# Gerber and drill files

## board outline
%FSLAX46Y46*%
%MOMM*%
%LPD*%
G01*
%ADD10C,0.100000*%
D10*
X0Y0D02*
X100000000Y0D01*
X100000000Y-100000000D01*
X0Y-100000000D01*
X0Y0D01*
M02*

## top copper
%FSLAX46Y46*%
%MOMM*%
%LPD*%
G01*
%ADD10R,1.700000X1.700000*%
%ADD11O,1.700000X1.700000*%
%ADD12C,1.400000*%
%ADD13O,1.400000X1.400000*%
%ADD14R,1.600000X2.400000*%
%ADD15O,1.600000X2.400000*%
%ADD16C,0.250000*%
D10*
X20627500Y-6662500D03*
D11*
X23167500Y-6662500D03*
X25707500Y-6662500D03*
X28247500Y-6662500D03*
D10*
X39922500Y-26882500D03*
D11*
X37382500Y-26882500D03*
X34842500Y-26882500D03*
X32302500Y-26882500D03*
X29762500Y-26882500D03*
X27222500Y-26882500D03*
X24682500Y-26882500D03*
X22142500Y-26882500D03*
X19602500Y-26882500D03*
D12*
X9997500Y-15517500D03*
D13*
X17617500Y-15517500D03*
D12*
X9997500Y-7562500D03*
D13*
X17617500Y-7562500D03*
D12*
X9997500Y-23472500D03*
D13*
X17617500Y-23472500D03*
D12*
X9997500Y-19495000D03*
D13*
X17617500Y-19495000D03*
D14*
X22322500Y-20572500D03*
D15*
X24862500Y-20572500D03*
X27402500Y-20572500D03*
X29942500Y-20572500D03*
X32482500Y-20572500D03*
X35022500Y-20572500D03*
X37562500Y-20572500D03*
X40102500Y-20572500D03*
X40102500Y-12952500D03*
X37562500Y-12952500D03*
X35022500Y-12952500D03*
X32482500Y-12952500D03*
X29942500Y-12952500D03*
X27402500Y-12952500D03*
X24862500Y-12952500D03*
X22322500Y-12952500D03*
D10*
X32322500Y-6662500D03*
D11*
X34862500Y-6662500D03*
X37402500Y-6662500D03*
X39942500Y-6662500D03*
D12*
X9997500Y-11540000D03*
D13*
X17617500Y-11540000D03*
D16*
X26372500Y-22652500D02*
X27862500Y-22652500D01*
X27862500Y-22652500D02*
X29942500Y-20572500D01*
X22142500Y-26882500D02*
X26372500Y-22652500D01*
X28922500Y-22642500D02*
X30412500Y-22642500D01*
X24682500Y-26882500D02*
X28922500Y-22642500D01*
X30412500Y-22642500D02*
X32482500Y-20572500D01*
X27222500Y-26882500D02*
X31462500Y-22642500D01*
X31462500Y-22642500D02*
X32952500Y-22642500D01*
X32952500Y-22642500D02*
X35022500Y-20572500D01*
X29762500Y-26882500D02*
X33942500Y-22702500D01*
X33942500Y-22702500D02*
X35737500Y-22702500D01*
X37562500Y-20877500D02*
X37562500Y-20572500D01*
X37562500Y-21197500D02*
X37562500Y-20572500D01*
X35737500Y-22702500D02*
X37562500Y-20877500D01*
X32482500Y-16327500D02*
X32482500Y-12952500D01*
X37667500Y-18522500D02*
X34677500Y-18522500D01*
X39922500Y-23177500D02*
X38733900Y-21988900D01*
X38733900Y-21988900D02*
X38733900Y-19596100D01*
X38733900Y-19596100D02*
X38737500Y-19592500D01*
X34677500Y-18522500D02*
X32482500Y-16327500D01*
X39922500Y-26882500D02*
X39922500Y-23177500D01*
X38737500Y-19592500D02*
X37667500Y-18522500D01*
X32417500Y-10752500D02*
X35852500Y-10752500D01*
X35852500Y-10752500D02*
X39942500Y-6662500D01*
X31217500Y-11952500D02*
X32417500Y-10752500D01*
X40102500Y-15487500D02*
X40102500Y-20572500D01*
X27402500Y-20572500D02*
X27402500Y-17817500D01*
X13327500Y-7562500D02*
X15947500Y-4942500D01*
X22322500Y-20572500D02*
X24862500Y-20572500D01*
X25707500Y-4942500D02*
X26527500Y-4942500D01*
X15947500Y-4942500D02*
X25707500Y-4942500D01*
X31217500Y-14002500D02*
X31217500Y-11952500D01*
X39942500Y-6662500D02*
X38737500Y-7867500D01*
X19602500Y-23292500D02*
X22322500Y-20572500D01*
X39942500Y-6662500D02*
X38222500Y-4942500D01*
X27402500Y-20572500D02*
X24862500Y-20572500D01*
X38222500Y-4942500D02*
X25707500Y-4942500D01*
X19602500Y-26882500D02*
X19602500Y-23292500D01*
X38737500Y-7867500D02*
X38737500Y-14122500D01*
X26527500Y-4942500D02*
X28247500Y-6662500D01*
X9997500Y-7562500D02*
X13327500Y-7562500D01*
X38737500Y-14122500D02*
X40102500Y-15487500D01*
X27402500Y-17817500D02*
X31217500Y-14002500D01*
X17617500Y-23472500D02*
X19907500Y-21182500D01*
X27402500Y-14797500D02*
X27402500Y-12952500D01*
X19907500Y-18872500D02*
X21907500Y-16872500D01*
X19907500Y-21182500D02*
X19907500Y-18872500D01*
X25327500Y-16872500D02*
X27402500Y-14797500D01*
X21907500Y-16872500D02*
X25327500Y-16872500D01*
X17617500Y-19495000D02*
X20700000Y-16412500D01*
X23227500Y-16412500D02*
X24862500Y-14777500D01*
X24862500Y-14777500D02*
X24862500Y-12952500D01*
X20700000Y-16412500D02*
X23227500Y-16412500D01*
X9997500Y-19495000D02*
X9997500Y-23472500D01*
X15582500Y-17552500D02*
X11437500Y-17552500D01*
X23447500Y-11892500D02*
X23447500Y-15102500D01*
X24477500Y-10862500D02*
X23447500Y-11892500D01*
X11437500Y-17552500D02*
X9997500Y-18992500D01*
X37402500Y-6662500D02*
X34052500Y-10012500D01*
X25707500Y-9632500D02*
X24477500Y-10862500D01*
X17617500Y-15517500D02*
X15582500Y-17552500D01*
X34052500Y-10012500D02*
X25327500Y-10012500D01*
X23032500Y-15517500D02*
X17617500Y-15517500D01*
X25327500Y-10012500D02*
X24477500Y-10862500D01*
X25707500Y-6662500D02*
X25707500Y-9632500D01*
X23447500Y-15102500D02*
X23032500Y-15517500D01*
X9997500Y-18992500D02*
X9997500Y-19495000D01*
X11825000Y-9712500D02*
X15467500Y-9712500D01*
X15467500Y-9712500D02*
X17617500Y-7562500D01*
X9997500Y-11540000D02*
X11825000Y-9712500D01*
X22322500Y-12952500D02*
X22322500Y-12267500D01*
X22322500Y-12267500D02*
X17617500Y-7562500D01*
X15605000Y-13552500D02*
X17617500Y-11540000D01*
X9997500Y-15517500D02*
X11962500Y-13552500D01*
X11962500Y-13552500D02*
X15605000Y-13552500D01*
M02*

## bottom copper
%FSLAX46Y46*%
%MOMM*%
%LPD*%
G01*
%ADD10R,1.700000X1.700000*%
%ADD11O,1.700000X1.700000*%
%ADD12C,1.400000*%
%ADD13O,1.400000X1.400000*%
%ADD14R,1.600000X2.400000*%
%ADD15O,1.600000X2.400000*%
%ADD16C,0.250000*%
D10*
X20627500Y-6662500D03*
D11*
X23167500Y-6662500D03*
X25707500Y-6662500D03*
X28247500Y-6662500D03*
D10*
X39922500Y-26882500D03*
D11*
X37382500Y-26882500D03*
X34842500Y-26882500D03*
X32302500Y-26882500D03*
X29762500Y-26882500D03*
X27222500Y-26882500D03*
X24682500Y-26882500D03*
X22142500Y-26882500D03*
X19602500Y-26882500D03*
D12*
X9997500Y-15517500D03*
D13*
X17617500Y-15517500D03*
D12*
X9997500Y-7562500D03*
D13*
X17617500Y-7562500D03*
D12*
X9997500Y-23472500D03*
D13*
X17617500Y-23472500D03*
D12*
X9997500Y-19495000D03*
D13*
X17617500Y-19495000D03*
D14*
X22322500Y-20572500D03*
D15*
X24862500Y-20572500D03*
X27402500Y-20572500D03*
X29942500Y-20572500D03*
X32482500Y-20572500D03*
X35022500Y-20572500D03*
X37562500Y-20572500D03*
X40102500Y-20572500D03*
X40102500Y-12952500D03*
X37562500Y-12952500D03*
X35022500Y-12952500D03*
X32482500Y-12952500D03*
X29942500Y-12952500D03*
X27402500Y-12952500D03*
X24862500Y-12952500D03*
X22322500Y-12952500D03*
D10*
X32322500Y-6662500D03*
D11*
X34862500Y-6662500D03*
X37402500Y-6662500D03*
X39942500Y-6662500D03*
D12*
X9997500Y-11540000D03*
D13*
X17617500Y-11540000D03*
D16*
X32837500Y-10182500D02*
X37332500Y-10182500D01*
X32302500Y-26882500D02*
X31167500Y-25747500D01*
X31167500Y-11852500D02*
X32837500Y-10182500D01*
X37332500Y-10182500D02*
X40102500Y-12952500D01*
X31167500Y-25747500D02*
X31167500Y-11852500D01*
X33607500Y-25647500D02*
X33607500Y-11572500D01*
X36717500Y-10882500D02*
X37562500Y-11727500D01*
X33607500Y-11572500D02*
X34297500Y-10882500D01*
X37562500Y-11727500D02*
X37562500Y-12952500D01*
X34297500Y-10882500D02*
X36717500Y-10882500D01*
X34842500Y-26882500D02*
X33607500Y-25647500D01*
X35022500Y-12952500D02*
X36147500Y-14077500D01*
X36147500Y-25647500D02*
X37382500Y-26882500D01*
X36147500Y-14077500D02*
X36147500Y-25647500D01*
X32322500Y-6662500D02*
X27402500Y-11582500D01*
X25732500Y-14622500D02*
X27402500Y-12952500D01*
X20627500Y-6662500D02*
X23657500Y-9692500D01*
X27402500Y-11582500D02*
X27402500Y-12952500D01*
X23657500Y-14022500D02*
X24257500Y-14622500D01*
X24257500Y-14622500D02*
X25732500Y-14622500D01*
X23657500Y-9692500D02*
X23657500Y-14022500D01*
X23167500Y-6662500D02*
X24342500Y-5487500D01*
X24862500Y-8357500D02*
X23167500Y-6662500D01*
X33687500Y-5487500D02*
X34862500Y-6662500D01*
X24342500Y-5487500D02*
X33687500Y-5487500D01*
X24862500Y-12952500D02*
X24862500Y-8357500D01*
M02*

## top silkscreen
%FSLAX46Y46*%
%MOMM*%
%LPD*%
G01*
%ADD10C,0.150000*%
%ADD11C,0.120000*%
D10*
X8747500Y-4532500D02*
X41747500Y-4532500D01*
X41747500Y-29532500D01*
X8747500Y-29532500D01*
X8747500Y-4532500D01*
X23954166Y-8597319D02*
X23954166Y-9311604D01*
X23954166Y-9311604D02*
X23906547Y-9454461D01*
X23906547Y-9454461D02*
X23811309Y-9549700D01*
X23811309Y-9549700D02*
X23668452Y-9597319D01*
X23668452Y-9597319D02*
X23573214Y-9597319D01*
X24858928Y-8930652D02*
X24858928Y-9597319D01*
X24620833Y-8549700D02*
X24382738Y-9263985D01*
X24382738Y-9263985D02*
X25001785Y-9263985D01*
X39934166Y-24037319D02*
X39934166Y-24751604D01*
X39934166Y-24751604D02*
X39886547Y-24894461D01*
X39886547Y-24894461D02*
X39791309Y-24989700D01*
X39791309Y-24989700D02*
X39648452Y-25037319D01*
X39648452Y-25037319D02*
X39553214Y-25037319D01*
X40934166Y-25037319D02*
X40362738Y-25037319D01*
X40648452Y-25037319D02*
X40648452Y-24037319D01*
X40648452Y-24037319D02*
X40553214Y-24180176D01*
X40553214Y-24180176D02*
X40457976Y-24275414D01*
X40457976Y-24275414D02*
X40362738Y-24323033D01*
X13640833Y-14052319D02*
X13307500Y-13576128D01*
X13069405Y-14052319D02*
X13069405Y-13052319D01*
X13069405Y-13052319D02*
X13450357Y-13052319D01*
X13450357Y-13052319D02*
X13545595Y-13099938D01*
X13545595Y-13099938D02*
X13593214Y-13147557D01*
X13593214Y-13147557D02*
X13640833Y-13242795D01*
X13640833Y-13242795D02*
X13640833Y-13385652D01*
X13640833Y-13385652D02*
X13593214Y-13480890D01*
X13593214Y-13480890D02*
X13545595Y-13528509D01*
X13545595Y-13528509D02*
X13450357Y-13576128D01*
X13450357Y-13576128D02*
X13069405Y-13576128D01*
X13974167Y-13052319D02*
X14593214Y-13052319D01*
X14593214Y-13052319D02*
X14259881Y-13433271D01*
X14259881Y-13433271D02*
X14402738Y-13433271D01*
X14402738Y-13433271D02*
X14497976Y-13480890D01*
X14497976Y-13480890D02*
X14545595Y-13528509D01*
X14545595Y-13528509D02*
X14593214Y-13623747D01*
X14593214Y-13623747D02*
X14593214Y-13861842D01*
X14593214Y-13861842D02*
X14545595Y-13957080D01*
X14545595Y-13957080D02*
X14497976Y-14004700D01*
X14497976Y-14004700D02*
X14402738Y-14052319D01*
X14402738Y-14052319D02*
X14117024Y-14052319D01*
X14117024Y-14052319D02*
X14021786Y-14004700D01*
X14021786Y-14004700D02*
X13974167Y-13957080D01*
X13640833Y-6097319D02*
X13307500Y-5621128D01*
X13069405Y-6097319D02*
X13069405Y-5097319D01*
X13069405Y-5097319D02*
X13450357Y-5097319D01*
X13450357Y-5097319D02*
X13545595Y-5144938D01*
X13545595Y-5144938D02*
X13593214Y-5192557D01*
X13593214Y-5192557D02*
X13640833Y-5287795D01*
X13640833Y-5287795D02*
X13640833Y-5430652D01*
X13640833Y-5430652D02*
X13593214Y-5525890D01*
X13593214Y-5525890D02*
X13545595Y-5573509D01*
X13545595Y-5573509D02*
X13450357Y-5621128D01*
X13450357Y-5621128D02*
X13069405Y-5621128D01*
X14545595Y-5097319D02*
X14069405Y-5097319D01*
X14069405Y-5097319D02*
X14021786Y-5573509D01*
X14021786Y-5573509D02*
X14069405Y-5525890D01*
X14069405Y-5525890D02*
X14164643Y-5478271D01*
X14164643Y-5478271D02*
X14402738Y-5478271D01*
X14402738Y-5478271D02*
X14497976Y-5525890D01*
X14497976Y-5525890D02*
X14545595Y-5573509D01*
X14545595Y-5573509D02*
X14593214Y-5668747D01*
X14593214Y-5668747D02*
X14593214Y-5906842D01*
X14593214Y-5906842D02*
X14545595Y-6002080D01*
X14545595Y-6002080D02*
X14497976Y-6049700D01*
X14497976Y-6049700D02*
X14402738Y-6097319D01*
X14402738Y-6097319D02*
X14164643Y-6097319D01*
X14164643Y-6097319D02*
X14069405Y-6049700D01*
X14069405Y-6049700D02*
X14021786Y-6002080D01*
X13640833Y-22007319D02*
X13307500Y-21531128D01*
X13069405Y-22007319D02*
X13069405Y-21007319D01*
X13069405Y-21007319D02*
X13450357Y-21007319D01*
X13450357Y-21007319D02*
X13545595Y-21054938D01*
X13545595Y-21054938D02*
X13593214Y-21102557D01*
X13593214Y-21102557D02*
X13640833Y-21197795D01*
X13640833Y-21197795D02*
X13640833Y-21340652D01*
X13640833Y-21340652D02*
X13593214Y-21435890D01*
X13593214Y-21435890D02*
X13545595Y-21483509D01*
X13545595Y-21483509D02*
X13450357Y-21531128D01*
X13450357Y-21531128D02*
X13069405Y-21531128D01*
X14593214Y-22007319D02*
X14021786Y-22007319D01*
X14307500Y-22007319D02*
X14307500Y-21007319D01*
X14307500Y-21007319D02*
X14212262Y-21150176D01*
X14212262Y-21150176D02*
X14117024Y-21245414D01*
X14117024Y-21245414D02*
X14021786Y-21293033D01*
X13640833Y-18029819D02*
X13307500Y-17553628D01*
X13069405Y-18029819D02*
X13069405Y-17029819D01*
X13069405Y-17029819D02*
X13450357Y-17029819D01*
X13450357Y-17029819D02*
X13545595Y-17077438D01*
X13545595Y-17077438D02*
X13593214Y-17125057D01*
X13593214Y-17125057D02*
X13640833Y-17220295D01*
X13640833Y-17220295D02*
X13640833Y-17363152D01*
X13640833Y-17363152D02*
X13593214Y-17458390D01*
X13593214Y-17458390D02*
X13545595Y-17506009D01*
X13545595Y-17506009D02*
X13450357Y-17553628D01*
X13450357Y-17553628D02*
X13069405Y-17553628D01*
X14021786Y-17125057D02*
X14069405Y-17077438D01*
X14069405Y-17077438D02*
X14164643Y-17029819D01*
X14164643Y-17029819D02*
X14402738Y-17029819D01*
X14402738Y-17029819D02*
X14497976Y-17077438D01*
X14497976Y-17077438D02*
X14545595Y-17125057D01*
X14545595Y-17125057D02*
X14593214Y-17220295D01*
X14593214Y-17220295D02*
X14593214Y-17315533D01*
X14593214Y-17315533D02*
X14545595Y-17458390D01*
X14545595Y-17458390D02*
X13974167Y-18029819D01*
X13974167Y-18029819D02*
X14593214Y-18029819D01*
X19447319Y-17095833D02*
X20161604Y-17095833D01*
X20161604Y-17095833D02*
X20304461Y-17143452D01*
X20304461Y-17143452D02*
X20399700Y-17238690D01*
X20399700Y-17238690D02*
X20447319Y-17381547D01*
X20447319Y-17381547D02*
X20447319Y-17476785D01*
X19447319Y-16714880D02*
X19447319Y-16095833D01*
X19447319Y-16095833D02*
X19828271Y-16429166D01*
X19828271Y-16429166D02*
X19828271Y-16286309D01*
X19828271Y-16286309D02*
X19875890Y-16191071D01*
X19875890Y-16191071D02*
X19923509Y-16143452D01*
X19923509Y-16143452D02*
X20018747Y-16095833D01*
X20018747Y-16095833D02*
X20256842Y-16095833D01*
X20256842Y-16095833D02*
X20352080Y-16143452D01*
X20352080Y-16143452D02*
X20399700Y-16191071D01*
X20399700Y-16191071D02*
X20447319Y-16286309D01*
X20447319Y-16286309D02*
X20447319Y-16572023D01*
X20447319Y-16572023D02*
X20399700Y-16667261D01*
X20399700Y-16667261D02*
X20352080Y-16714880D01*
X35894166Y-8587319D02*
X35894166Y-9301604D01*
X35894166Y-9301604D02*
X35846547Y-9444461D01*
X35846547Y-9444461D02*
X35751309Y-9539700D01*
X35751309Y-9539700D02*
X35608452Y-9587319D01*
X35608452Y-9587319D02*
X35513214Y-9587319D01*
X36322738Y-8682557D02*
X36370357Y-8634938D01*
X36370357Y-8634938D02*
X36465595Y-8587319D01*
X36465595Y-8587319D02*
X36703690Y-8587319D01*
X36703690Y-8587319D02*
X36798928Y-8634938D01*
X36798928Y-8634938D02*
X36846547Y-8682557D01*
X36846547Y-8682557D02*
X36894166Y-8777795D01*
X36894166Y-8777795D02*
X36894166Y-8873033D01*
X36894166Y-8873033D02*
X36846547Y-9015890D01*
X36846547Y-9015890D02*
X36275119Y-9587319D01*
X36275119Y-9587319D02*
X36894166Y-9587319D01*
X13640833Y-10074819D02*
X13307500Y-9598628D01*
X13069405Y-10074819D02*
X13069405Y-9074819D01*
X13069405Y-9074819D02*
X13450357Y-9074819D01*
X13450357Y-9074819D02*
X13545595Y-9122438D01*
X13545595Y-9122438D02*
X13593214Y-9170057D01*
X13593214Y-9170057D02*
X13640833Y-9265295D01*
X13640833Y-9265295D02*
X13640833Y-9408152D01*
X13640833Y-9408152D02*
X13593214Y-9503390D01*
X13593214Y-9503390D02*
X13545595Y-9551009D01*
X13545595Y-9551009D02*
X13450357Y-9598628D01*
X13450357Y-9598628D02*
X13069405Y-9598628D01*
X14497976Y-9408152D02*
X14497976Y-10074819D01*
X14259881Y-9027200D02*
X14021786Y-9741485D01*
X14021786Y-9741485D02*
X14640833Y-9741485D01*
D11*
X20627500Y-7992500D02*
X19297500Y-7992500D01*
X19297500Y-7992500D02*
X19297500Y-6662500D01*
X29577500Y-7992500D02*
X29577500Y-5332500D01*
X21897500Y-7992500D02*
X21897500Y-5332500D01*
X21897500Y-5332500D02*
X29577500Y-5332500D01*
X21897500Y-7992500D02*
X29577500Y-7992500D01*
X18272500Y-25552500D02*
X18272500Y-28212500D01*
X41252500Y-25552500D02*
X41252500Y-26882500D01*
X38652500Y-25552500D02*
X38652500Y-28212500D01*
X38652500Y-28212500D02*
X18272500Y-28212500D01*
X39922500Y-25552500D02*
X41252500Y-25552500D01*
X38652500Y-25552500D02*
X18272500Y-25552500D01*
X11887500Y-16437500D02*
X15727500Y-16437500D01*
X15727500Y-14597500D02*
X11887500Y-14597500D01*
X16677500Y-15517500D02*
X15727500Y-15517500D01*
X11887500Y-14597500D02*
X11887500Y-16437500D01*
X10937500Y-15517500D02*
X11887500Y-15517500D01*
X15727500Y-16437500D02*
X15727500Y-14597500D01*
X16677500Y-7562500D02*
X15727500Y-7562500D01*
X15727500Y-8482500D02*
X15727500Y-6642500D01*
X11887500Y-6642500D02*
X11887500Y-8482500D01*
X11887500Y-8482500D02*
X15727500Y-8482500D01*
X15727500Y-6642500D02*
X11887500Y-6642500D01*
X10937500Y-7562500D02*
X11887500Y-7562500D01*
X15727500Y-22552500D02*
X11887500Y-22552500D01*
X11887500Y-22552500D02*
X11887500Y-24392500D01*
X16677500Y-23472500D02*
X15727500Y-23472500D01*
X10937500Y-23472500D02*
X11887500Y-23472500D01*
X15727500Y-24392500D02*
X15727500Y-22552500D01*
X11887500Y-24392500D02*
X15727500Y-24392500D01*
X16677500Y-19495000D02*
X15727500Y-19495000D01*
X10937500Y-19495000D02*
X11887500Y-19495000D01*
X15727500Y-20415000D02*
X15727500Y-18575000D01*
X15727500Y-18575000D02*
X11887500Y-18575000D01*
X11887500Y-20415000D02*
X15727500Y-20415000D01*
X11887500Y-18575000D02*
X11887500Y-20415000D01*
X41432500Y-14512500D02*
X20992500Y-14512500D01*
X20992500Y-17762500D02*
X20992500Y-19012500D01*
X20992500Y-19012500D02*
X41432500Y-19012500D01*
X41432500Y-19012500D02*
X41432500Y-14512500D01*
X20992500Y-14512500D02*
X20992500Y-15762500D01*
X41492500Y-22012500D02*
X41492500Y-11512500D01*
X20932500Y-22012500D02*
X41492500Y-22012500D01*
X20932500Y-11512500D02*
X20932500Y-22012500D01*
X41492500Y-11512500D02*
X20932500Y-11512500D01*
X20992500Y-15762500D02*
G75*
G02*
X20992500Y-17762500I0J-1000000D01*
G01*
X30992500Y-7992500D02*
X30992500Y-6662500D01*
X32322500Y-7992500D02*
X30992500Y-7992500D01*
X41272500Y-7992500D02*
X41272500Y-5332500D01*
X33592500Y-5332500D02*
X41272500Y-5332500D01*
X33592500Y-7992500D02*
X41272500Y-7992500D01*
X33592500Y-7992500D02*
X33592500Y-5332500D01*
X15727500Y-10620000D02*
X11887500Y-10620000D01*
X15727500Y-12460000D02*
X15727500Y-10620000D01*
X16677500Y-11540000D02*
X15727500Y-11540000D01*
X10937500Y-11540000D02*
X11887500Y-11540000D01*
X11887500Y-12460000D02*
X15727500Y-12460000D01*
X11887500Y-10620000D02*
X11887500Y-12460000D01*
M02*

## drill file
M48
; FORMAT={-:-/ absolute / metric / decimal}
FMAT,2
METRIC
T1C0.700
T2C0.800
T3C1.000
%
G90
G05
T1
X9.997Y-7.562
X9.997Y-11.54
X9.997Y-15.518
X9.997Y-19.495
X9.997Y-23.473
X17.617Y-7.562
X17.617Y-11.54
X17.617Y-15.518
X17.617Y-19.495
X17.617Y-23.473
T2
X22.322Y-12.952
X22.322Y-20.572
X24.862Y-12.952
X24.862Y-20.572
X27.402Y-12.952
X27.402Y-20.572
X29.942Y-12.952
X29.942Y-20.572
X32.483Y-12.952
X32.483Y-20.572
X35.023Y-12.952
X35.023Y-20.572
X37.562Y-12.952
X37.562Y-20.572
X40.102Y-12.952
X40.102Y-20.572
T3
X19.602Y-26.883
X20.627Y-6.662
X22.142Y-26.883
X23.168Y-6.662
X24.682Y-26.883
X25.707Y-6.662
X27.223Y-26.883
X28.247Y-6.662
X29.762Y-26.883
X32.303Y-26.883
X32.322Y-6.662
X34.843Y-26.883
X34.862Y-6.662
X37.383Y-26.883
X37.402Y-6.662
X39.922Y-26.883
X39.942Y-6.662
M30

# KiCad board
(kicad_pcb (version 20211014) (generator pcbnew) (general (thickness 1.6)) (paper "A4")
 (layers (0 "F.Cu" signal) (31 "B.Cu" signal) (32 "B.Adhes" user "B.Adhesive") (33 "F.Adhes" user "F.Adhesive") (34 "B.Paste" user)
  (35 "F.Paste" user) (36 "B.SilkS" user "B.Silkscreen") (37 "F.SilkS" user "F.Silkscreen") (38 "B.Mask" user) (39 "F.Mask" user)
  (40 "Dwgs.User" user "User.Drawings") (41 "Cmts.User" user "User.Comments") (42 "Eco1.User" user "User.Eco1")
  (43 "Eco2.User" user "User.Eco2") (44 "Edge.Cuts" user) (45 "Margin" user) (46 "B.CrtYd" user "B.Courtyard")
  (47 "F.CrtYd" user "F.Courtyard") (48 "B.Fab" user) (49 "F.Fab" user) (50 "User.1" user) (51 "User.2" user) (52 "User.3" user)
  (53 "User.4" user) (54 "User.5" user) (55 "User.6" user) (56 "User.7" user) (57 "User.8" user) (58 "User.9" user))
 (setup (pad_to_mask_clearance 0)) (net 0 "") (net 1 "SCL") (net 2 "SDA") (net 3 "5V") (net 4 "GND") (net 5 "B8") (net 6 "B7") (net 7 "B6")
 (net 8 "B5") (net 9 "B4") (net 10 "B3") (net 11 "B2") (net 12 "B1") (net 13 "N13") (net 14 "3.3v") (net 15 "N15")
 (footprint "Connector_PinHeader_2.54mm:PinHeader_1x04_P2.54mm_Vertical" (layer "F.Cu") (at 20.6275 6.6625 90)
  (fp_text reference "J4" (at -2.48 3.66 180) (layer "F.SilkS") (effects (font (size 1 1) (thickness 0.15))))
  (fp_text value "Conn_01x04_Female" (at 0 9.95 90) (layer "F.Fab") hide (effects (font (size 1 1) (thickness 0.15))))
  (fp_line (start -1.33 0) (end -1.33 -1.33) (layer "F.SilkS") (width 0.12))
  (fp_line (start -1.33 -1.33) (end 0 -1.33) (layer "F.SilkS") (width 0.12))
  (fp_line (start -1.33 8.95) (end 1.33 8.95) (layer "F.SilkS") (width 0.12))
  (fp_line (start -1.33 1.27) (end 1.33 1.27) (layer "F.SilkS") (width 0.12))
  (fp_line (start 1.33 1.27) (end 1.33 8.95) (layer "F.SilkS") (width 0.12))
  (fp_line (start -1.33 1.27) (end -1.33 8.95) (layer "F.SilkS") (width 0.12))
  (pad "1" thru_hole rect (at 0 0 90) (size 1.7 1.7) (drill 1) (layers *.Cu *.Mask) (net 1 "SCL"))
  (pad "2" thru_hole oval (at 0 2.54 90) (size 1.7 1.7) (drill 1) (layers *.Cu *.Mask) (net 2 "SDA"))
  (pad "3" thru_hole oval (at 0 5.08 90) (size 1.7 1.7) (drill 1) (layers *.Cu *.Mask) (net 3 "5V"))
  (pad "4" thru_hole oval (at 0 7.62 90) (size 1.7 1.7) (drill 1) (layers *.Cu *.Mask) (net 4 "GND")))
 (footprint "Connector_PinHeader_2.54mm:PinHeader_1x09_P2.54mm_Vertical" (layer "F.Cu") (at 39.9225 26.8825 -90)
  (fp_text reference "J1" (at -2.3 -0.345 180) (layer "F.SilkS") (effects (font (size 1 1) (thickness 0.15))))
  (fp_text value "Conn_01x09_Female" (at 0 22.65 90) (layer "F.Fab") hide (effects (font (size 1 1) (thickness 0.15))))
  (fp_line (start -1.33 21.65) (end 1.33 21.65) (layer "F.SilkS") (width 0.12))
  (fp_line (start -1.33 -1.33) (end 0 -1.33) (layer "F.SilkS") (width 0.12))
  (fp_line (start -1.33 1.27) (end 1.33 1.27) (layer "F.SilkS") (width 0.12))
  (fp_line (start 1.33 1.27) (end 1.33 21.65) (layer "F.SilkS") (width 0.12))
  (fp_line (start -1.33 0) (end -1.33 -1.33) (layer "F.SilkS") (width 0.12))
  (fp_line (start -1.33 1.27) (end -1.33 21.65) (layer "F.SilkS") (width 0.12))
  (pad "1" thru_hole rect (at 0 0 270) (size 1.7 1.7) (drill 1) (layers *.Cu *.Mask) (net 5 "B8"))
  (pad "2" thru_hole oval (at 0 2.54 270) (size 1.7 1.7) (drill 1) (layers *.Cu *.Mask) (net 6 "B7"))
  (pad "3" thru_hole oval (at 0 5.08 270) (size 1.7 1.7) (drill 1) (layers *.Cu *.Mask) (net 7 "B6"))
  (pad "4" thru_hole oval (at 0 7.62 270) (size 1.7 1.7) (drill 1) (layers *.Cu *.Mask) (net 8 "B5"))
  (pad "5" thru_hole oval (at 0 10.16 270) (size 1.7 1.7) (drill 1) (layers *.Cu *.Mask) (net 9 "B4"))
  (pad "6" thru_hole oval (at 0 12.7 270) (size 1.7 1.7) (drill 1) (layers *.Cu *.Mask) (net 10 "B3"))
  (pad "7" thru_hole oval (at 0 15.24 270) (size 1.7 1.7) (drill 1) (layers *.Cu *.Mask) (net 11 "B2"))
  (pad "8" thru_hole oval (at 0 17.78 270) (size 1.7 1.7) (drill 1) (layers *.Cu *.Mask) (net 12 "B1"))
  (pad "9" thru_hole oval (at 0 20.32 270) (size 1.7 1.7) (drill 1) (layers *.Cu *.Mask) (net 4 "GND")))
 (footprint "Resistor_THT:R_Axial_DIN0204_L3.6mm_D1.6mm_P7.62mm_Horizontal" (layer "F.Cu") (at 9.9975 15.5175)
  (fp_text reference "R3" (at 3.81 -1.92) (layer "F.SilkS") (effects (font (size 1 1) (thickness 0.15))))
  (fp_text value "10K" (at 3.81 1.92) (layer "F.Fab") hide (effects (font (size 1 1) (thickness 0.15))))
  (fp_line (start 1.89 0.92) (end 5.73 0.92) (layer "F.SilkS") (width 0.12))
  (fp_line (start 5.73 -0.92) (end 1.89 -0.92) (layer "F.SilkS") (width 0.12))
  (fp_line (start 6.68 0) (end 5.73 0) (layer "F.SilkS") (width 0.12))
  (fp_line (start 1.89 -0.92) (end 1.89 0.92) (layer "F.SilkS") (width 0.12))
  (fp_line (start 0.94 0) (end 1.89 0) (layer "F.SilkS") (width 0.12))
  (fp_line (start 5.73 0.92) (end 5.73 -0.92) (layer "F.SilkS") (width 0.12))
  (pad "1" thru_hole circle (at 0 0) (size 1.4 1.4) (drill 0.7) (layers *.Cu *.Mask) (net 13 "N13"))
  (pad "2" thru_hole oval (at 7.62 0) (size 1.4 1.4) (drill 0.7) (layers *.Cu *.Mask) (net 3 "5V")))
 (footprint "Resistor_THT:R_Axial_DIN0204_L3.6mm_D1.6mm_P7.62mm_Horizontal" (layer "F.Cu") (at 9.9975 7.5625)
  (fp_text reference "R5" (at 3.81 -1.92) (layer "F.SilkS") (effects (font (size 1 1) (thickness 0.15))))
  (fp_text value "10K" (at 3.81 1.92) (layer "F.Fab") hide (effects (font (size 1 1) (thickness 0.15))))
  (fp_line (start 6.68 0) (end 5.73 0) (layer "F.SilkS") (width 0.12))
  (fp_line (start 5.73 0.92) (end 5.73 -0.92) (layer "F.SilkS") (width 0.12))
  (fp_line (start 1.89 -0.92) (end 1.89 0.92) (layer "F.SilkS") (width 0.12))
  (fp_line (start 1.89 0.92) (end 5.73 0.92) (layer "F.SilkS") (width 0.12))
  (fp_line (start 5.73 -0.92) (end 1.89 -0.92) (layer "F.SilkS") (width 0.12))
  (fp_line (start 0.94 0) (end 1.89 0) (layer "F.SilkS") (width 0.12))
  (pad "1" thru_hole circle (at 0 0) (size 1.4 1.4) (drill 0.7) (layers *.Cu *.Mask) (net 4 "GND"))
  (pad "2" thru_hole oval (at 7.62 0) (size 1.4 1.4) (drill 0.7) (layers *.Cu *.Mask) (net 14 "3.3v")))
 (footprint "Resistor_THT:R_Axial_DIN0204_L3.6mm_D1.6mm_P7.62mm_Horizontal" (layer "F.Cu") (at 9.9975 23.4725)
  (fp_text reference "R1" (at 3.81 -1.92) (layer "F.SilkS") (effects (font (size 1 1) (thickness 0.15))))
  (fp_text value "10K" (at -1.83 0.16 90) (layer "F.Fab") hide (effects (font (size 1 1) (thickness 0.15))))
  (fp_line (start 5.73 -0.92) (end 1.89 -0.92) (layer "F.SilkS") (width 0.12))
  (fp_line (start 1.89 -0.92) (end 1.89 0.92) (layer "F.SilkS") (width 0.12))
  (fp_line (start 6.68 0) (end 5.73 0) (layer "F.SilkS") (width 0.12))
  (fp_line (start 0.94 0) (end 1.89 0) (layer "F.SilkS") (width 0.12))
  (fp_line (start 5.73 0.92) (end 5.73 -0.92) (layer "F.SilkS") (width 0.12))
  (fp_line (start 1.89 0.92) (end 5.73 0.92) (layer "F.SilkS") (width 0.12))
  (pad "1" thru_hole circle (at 0 0) (size 1.4 1.4) (drill 0.7) (layers *.Cu *.Mask) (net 3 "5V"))
  (pad "2" thru_hole oval (at 7.62 0) (size 1.4 1.4) (drill 0.7) (layers *.Cu *.Mask) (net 1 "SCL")))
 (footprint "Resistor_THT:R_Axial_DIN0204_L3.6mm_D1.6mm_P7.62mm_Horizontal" (layer "F.Cu") (at 9.9975 19.495)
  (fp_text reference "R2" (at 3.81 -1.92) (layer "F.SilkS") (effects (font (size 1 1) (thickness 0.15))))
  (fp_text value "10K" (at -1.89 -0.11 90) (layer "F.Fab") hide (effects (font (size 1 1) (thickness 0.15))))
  (fp_line (start 6.68 0) (end 5.73 0) (layer "F.SilkS") (width 0.12))
  (fp_line (start 0.94 0) (end 1.89 0) (layer "F.SilkS") (width 0.12))
  (fp_line (start 5.73 0.92) (end 5.73 -0.92) (layer "F.SilkS") (width 0.12))
  (fp_line (start 5.73 -0.92) (end 1.89 -0.92) (layer "F.SilkS") (width 0.12))
  (fp_line (start 1.89 0.92) (end 5.73 0.92) (layer "F.SilkS") (width 0.12))
  (fp_line (start 1.89 -0.92) (end 1.89 0.92) (layer "F.SilkS") (width 0.12))
  (pad "1" thru_hole circle (at 0 0) (size 1.4 1.4) (drill 0.7) (layers *.Cu *.Mask) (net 3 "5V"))
  (pad "2" thru_hole oval (at 7.62 0) (size 1.4 1.4) (drill 0.7) (layers *.Cu *.Mask) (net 2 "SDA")))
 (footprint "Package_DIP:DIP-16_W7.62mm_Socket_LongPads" (layer "F.Cu") (at 22.3225 20.5725 90)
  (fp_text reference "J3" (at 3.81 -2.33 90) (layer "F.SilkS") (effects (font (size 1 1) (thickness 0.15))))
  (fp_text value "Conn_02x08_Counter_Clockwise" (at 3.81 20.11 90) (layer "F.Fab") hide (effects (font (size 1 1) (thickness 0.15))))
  (fp_line (start 6.06 19.11) (end 6.06 -1.33) (layer "F.SilkS") (width 0.12))
  (fp_line (start 2.81 -1.33) (end 1.56 -1.33) (layer "F.SilkS") (width 0.12))
  (fp_line (start 1.56 -1.33) (end 1.56 19.11) (layer "F.SilkS") (width 0.12))
  (fp_line (start 1.56 19.11) (end 6.06 19.11) (layer "F.SilkS") (width 0.12))
  (fp_line (start 6.06 -1.33) (end 4.81 -1.33) (layer "F.SilkS") (width 0.12))
  (fp_line (start -1.44 19.17) (end 9.06 19.17) (layer "F.SilkS") (width 0.12))
  (fp_line (start -1.44 -1.39) (end -1.44 19.17) (layer "F.SilkS") (width 0.12))
  (fp_line (start 9.06 -1.39) (end -1.44 -1.39) (layer "F.SilkS") (width 0.12))
  (fp_line (start 9.06 19.17) (end 9.06 -1.39) (layer "F.SilkS") (width 0.12))
  (fp_arc (start 4.81 -1.33) (mid 3.81 -0.33) (end 2.81 -1.33) (layer "F.SilkS") (width 0.12))
  (pad "1" thru_hole rect (at 0 0 90) (size 2.4 1.6) (drill 0.8) (layers *.Cu *.Mask) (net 4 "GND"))
  (pad "2" thru_hole oval (at 0 2.54 90) (size 2.4 1.6) (drill 0.8) (layers *.Cu *.Mask) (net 4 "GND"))
  (pad "3" thru_hole oval (at 0 5.08 90) (size 2.4 1.6) (drill 0.8) (layers *.Cu *.Mask) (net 4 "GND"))
  (pad "4" thru_hole oval (at 0 7.62 90) (size 2.4 1.6) (drill 0.8) (layers *.Cu *.Mask) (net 12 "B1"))
  (pad "5" thru_hole oval (at 0 10.16 90) (size 2.4 1.6) (drill 0.8) (layers *.Cu *.Mask) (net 11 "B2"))
  (pad "6" thru_hole oval (at 0 12.7 90) (size 2.4 1.6) (drill 0.8) (layers *.Cu *.Mask) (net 10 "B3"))
  (pad "7" thru_hole oval (at 0 15.24 90) (size 2.4 1.6) (drill 0.8) (layers *.Cu *.Mask) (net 9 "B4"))
  (pad "8" thru_hole oval (at 0 17.78 90) (size 2.4 1.6) (drill 0.8) (layers *.Cu *.Mask) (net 4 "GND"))
  (pad "9" thru_hole oval (at 7.62 17.78 90) (size 2.4 1.6) (drill 0.8) (layers *.Cu *.Mask) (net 8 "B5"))
  (pad "10" thru_hole oval (at 7.62 15.24 90) (size 2.4 1.6) (drill 0.8) (layers *.Cu *.Mask) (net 7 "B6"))
  (pad "11" thru_hole oval (at 7.62 12.7 90) (size 2.4 1.6) (drill 0.8) (layers *.Cu *.Mask) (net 6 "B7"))
  (pad "12" thru_hole oval (at 7.62 10.16 90) (size 2.4 1.6) (drill 0.8) (layers *.Cu *.Mask) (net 5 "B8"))
  (pad "13" thru_hole oval (at 7.62 7.62 90) (size 2.4 1.6) (drill 0.8) (layers *.Cu *.Mask) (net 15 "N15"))
  (pad "14" thru_hole oval (at 7.62 5.08 90) (size 2.4 1.6) (drill 0.8) (layers *.Cu *.Mask) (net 1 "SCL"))
  (pad "15" thru_hole oval (at 7.62 2.54 90) (size 2.4 1.6) (drill 0.8) (layers *.Cu *.Mask) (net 2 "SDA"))
  (pad "16" thru_hole oval (at 7.62 0 90) (size 2.4 1.6) (drill 0.8) (layers *.Cu *.Mask) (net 14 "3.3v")))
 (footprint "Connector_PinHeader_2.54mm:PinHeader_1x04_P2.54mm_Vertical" (layer "F.Cu") (at 32.3225 6.6625 90)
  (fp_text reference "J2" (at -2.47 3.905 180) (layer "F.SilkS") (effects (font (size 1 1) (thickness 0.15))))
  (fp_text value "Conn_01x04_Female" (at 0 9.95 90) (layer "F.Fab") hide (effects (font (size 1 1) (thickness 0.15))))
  (fp_line (start -1.33 -1.33) (end 0 -1.33) (layer "F.SilkS") (width 0.12))
  (fp_line (start -1.33 0) (end -1.33 -1.33) (layer "F.SilkS") (width 0.12))
  (fp_line (start -1.33 8.95) (end 1.33 8.95) (layer "F.SilkS") (width 0.12))
  (fp_line (start 1.33 1.27) (end 1.33 8.95) (layer "F.SilkS") (width 0.12))
  (fp_line (start -1.33 1.27) (end -1.33 8.95) (layer "F.SilkS") (width 0.12))
  (fp_line (start -1.33 1.27) (end 1.33 1.27) (layer "F.SilkS") (width 0.12))
  (pad "1" thru_hole rect (at 0 0 90) (size 1.7 1.7) (drill 1) (layers *.Cu *.Mask) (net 1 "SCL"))
  (pad "2" thru_hole oval (at 0 2.54 90) (size 1.7 1.7) (drill 1) (layers *.Cu *.Mask) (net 2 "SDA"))
  (pad "3" thru_hole oval (at 0 5.08 90) (size 1.7 1.7) (drill 1) (layers *.Cu *.Mask) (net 3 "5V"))
  (pad "4" thru_hole oval (at 0 7.62 90) (size 1.7 1.7) (drill 1) (layers *.Cu *.Mask) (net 4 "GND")))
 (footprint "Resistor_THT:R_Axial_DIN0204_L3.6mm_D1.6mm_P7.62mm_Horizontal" (layer "F.Cu") (at 9.9975 11.54)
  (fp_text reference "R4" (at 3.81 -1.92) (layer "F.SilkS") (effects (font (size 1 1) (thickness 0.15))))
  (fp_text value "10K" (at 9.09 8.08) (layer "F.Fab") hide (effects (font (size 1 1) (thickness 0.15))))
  (fp_line (start 5.73 -0.92) (end 1.89 -0.92) (layer "F.SilkS") (width 0.12))
  (fp_line (start 5.73 0.92) (end 5.73 -0.92) (layer "F.SilkS") (width 0.12))
  (fp_line (start 6.68 0) (end 5.73 0) (layer "F.SilkS") (width 0.12))
  (fp_line (start 0.94 0) (end 1.89 0) (layer "F.SilkS") (width 0.12))
  (fp_line (start 1.89 0.92) (end 5.73 0.92) (layer "F.SilkS") (width 0.12))
  (fp_line (start 1.89 -0.92) (end 1.89 0.92) (layer "F.SilkS") (width 0.12))
  (pad "1" thru_hole circle (at 0 0) (size 1.4 1.4) (drill 0.7) (layers *.Cu *.Mask) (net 14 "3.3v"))
  (pad "2" thru_hole oval (at 7.62 0) (size 1.4 1.4) (drill 0.7) (layers *.Cu *.Mask) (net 13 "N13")))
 (gr_rect (start 41.7475 29.5325) (end 8.7475 4.5325) (layer "F.SilkS") (width 0.15) (fill none))
 (gr_rect (start 0 0) (end 100 100) (layer "Edge.Cuts") (width 0.1) (fill none))
 (segment (start 26.3725 22.6525) (end 27.8625 22.6525) (width 0.25) (layer "F.Cu") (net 12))
 (segment (start 27.8625 22.6525) (end 29.9425 20.5725) (width 0.25) (layer "F.Cu") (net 12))
 (segment (start 22.1425 26.8825) (end 26.3725 22.6525) (width 0.25) (layer "F.Cu") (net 12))
 (segment (start 28.9225 22.6425) (end 30.4125 22.6425) (width 0.25) (layer "F.Cu") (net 11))
 (segment (start 24.6825 26.8825) (end 28.9225 22.6425) (width 0.25) (layer "F.Cu") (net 11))
 (segment (start 30.4125 22.6425) (end 32.4825 20.5725) (width 0.25) (layer "F.Cu") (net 11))
 (segment (start 27.2225 26.8825) (end 31.4625 22.6425) (width 0.25) (layer "F.Cu") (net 10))
 (segment (start 31.4625 22.6425) (end 32.9525 22.6425) (width 0.25) (layer "F.Cu") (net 10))
 (segment (start 32.9525 22.6425) (end 35.0225 20.5725) (width 0.25) (layer "F.Cu") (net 10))
 (segment (start 29.7625 26.8825) (end 33.9425 22.7025) (width 0.25) (layer "F.Cu") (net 9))
 (segment (start 33.9425 22.7025) (end 35.7375 22.7025) (width 0.25) (layer "F.Cu") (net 9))
 (segment (start 37.5625 20.8775) (end 37.5625 20.5725) (width 0.25) (layer "F.Cu") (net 9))
 (segment (start 37.5625 21.1975) (end 37.5625 20.5725) (width 0.25) (layer "F.Cu") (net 9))
 (segment (start 35.7375 22.7025) (end 37.5625 20.8775) (width 0.25) (layer "F.Cu") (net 9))
 (segment (start 32.8375 10.1825) (end 37.3325 10.1825) (width 0.25) (layer "B.Cu") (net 8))
 (segment (start 32.3025 26.8825) (end 31.1675 25.7475) (width 0.25) (layer "B.Cu") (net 8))
 (segment (start 31.1675 11.8525) (end 32.8375 10.1825) (width 0.25) (layer "B.Cu") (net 8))
 (segment (start 37.3325 10.1825) (end 40.1025 12.9525) (width 0.25) (layer "B.Cu") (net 8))
 (segment (start 31.1675 25.7475) (end 31.1675 11.8525) (width 0.25) (layer "B.Cu") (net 8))
 (segment (start 33.6075 25.6475) (end 33.6075 11.5725) (width 0.25) (layer "B.Cu") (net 7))
 (segment (start 36.7175 10.8825) (end 37.5625 11.7275) (width 0.25) (layer "B.Cu") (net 7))
 (segment (start 33.6075 11.5725) (end 34.2975 10.8825) (width 0.25) (layer "B.Cu") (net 7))
 (segment (start 37.5625 11.7275) (end 37.5625 12.9525) (width 0.25) (layer "B.Cu") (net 7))
 (segment (start 34.2975 10.8825) (end 36.7175 10.8825) (width 0.25) (layer "B.Cu") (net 7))
 (segment (start 34.8425 26.8825) (end 33.6075 25.6475) (width 0.25) (layer "B.Cu") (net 7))
 (segment (start 35.0225 12.9525) (end 36.1475 14.0775) (width 0.25) (layer "B.Cu") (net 6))
 (segment (start 36.1475 25.6475) (end 37.3825 26.8825) (width 0.25) (layer "B.Cu") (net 6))
 (segment (start 36.1475 14.0775) (end 36.1475 25.6475) (width 0.25) (layer "B.Cu") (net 6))
 (segment (start 32.4825 16.3275) (end 32.4825 12.9525) (width 0.25) (layer "F.Cu") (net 5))
 (segment (start 37.6675 18.5225) (end 34.6775 18.5225) (width 0.25) (layer "F.Cu") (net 5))
 (segment (start 39.9225 23.1775) (end 38.7339 21.9889) (width 0.25) (layer "F.Cu") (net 5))
 (segment (start 38.7339 21.9889) (end 38.7339 19.5961) (width 0.25) (layer "F.Cu") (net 5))
 (segment (start 38.7339 19.5961) (end 38.7375 19.5925) (width 0.25) (layer "F.Cu") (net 5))
 (segment (start 34.6775 18.5225) (end 32.4825 16.3275) (width 0.25) (layer "F.Cu") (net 5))
 (segment (start 39.9225 26.8825) (end 39.9225 23.1775) (width 0.25) (layer "F.Cu") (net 5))
 (segment (start 38.7375 19.5925) (end 37.6675 18.5225) (width 0.25) (layer "F.Cu") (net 5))
 (segment (start 32.4175 10.7525) (end 35.8525 10.7525) (width 0.25) (layer "F.Cu") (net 4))
 (segment (start 35.8525 10.7525) (end 39.9425 6.6625) (width 0.25) (layer "F.Cu") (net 4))
 (segment (start 31.2175 11.9525) (end 32.4175 10.7525) (width 0.25) (layer "F.Cu") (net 4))
 (segment (start 40.1025 15.4875) (end 40.1025 20.5725) (width 0.25) (layer "F.Cu") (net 4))
 (segment (start 27.4025 20.5725) (end 27.4025 17.8175) (width 0.25) (layer "F.Cu") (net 4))
 (segment (start 13.3275 7.5625) (end 15.9475 4.9425) (width 0.25) (layer "F.Cu") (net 4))
 (segment (start 22.3225 20.5725) (end 24.8625 20.5725) (width 0.25) (layer "F.Cu") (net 4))
 (segment (start 25.7075 4.9425) (end 26.5275 4.9425) (width 0.25) (layer "F.Cu") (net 4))
 (segment (start 15.9475 4.9425) (end 25.7075 4.9425) (width 0.25) (layer "F.Cu") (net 4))
 (segment (start 31.2175 14.0025) (end 31.2175 11.9525) (width 0.25) (layer "F.Cu") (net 4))
 (segment (start 39.9425 6.6625) (end 38.7375 7.8675) (width 0.25) (layer "F.Cu") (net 4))
 (segment (start 19.6025 23.2925) (end 22.3225 20.5725) (width 0.25) (layer "F.Cu") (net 4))
 (segment (start 39.9425 6.6625) (end 38.2225 4.9425) (width 0.25) (layer "F.Cu") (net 4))
 (segment (start 27.4025 20.5725) (end 24.8625 20.5725) (width 0.25) (layer "F.Cu") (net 4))
 (segment (start 38.2225 4.9425) (end 25.7075 4.9425) (width 0.25) (layer "F.Cu") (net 4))
 (segment (start 19.6025 26.8825) (end 19.6025 23.2925) (width 0.25) (layer "F.Cu") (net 4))
 (segment (start 38.7375 7.8675) (end 38.7375 14.1225) (width 0.25) (layer "F.Cu") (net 4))
 (segment (start 26.5275 4.9425) (end 28.2475 6.6625) (width 0.25) (layer "F.Cu") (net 4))
 (segment (start 9.9975 7.5625) (end 13.3275 7.5625) (width 0.25) (layer "F.Cu") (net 4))
 (segment (start 38.7375 14.1225) (end 40.1025 15.4875) (width 0.25) (layer "F.Cu") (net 4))
 (segment (start 27.4025 17.8175) (end 31.2175 14.0025) (width 0.25) (layer "F.Cu") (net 4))
 (segment (start 17.6175 23.4725) (end 19.9075 21.1825) (width 0.25) (layer "F.Cu") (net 1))
 (segment (start 27.4025 14.7975) (end 27.4025 12.9525) (width 0.25) (layer "F.Cu") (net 1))
 (segment (start 19.9075 18.8725) (end 21.9075 16.8725) (width 0.25) (layer "F.Cu") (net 1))
 (segment (start 19.9075 21.1825) (end 19.9075 18.8725) (width 0.25) (layer "F.Cu") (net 1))
 (segment (start 25.3275 16.8725) (end 27.4025 14.7975) (width 0.25) (layer "F.Cu") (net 1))
 (segment (start 21.9075 16.8725) (end 25.3275 16.8725) (width 0.25) (layer "F.Cu") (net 1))
 (segment (start 32.3225 6.6625) (end 27.4025 11.5825) (width 0.25) (layer "B.Cu") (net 1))
 (segment (start 25.7325 14.6225) (end 27.4025 12.9525) (width 0.25) (layer "B.Cu") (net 1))
 (segment (start 20.6275 6.6625) (end 23.6575 9.6925) (width 0.25) (layer "B.Cu") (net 1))
 (segment (start 27.4025 11.5825) (end 27.4025 12.9525) (width 0.25) (layer "B.Cu") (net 1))
 (segment (start 23.6575 14.0225) (end 24.2575 14.6225) (width 0.25) (layer "B.Cu") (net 1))
 (segment (start 24.2575 14.6225) (end 25.7325 14.6225) (width 0.25) (layer "B.Cu") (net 1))
 (segment (start 23.6575 9.6925) (end 23.6575 14.0225) (width 0.25) (layer "B.Cu") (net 1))
 (segment (start 17.6175 19.495) (end 20.7 16.4125) (width 0.25) (layer "F.Cu") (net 2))
 (segment (start 23.2275 16.4125) (end 24.8625 14.7775) (width 0.25) (layer "F.Cu") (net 2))
 (segment (start 24.8625 14.7775) (end 24.8625 12.9525) (width 0.25) (layer "F.Cu") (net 2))
 (segment (start 20.7 16.4125) (end 23.2275 16.4125) (width 0.25) (layer "F.Cu") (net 2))
 (segment (start 23.1675 6.6625) (end 24.3425 5.4875) (width 0.25) (layer "B.Cu") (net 2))
 (segment (start 24.8625 8.3575) (end 23.1675 6.6625) (width 0.25) (layer "B.Cu") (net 2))
 (segment (start 33.6875 5.4875) (end 34.8625 6.6625) (width 0.25) (layer "B.Cu") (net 2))
 (segment (start 24.3425 5.4875) (end 33.6875 5.4875) (width 0.25) (layer "B.Cu") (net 2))
 (segment (start 24.8625 12.9525) (end 24.8625 8.3575) (width 0.25) (layer "B.Cu") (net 2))
 (segment (start 9.9975 19.495) (end 9.9975 23.4725) (width 0.25) (layer "F.Cu") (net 3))
 (segment (start 15.5825 17.5525) (end 11.4375 17.5525) (width 0.25) (layer "F.Cu") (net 3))
 (segment (start 23.4475 11.8925) (end 23.4475 15.1025) (width 0.25) (layer "F.Cu") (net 3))
 (segment (start 24.4775 10.8625) (end 23.4475 11.8925) (width 0.25) (layer "F.Cu") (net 3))
 (segment (start 11.4375 17.5525) (end 9.9975 18.9925) (width 0.25) (layer "F.Cu") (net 3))
 (segment (start 37.4025 6.6625) (end 34.0525 10.0125) (width 0.25) (layer "F.Cu") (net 3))
 (segment (start 25.7075 9.6325) (end 24.4775 10.8625) (width 0.25) (layer "F.Cu") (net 3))
 (segment (start 17.6175 15.5175) (end 15.5825 17.5525) (width 0.25) (layer "F.Cu") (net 3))
 (segment (start 34.0525 10.0125) (end 25.3275 10.0125) (width 0.25) (layer "F.Cu") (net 3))
 (segment (start 23.0325 15.5175) (end 17.6175 15.5175) (width 0.25) (layer "F.Cu") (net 3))
 (segment (start 25.3275 10.0125) (end 24.4775 10.8625) (width 0.25) (layer "F.Cu") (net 3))
 (segment (start 25.7075 6.6625) (end 25.7075 9.6325) (width 0.25) (layer "F.Cu") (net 3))
 (segment (start 23.4475 15.1025) (end 23.0325 15.5175) (width 0.25) (layer "F.Cu") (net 3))
 (segment (start 9.9975 18.9925) (end 9.9975 19.495) (width 0.25) (layer "F.Cu") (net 3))
 (segment (start 11.825 9.7125) (end 15.4675 9.7125) (width 0.25) (layer "F.Cu") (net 14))
 (segment (start 15.4675 9.7125) (end 17.6175 7.5625) (width 0.25) (layer "F.Cu") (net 14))
 (segment (start 9.9975 11.54) (end 11.825 9.7125) (width 0.25) (layer "F.Cu") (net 14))
 (segment (start 22.3225 12.9525) (end 22.3225 12.2675) (width 0.25) (layer "F.Cu") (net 14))
 (segment (start 22.3225 12.2675) (end 17.6175 7.5625) (width 0.25) (layer "F.Cu") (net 14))
 (segment (start 15.605 13.5525) (end 17.6175 11.54) (width 0.25) (layer "F.Cu") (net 13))
 (segment (start 9.9975 15.5175) (end 11.9625 13.5525) (width 0.25) (layer "F.Cu") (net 13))
 (segment (start 11.9625 13.5525) (end 15.605 13.5525) (width 0.25) (layer "F.Cu") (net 13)))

